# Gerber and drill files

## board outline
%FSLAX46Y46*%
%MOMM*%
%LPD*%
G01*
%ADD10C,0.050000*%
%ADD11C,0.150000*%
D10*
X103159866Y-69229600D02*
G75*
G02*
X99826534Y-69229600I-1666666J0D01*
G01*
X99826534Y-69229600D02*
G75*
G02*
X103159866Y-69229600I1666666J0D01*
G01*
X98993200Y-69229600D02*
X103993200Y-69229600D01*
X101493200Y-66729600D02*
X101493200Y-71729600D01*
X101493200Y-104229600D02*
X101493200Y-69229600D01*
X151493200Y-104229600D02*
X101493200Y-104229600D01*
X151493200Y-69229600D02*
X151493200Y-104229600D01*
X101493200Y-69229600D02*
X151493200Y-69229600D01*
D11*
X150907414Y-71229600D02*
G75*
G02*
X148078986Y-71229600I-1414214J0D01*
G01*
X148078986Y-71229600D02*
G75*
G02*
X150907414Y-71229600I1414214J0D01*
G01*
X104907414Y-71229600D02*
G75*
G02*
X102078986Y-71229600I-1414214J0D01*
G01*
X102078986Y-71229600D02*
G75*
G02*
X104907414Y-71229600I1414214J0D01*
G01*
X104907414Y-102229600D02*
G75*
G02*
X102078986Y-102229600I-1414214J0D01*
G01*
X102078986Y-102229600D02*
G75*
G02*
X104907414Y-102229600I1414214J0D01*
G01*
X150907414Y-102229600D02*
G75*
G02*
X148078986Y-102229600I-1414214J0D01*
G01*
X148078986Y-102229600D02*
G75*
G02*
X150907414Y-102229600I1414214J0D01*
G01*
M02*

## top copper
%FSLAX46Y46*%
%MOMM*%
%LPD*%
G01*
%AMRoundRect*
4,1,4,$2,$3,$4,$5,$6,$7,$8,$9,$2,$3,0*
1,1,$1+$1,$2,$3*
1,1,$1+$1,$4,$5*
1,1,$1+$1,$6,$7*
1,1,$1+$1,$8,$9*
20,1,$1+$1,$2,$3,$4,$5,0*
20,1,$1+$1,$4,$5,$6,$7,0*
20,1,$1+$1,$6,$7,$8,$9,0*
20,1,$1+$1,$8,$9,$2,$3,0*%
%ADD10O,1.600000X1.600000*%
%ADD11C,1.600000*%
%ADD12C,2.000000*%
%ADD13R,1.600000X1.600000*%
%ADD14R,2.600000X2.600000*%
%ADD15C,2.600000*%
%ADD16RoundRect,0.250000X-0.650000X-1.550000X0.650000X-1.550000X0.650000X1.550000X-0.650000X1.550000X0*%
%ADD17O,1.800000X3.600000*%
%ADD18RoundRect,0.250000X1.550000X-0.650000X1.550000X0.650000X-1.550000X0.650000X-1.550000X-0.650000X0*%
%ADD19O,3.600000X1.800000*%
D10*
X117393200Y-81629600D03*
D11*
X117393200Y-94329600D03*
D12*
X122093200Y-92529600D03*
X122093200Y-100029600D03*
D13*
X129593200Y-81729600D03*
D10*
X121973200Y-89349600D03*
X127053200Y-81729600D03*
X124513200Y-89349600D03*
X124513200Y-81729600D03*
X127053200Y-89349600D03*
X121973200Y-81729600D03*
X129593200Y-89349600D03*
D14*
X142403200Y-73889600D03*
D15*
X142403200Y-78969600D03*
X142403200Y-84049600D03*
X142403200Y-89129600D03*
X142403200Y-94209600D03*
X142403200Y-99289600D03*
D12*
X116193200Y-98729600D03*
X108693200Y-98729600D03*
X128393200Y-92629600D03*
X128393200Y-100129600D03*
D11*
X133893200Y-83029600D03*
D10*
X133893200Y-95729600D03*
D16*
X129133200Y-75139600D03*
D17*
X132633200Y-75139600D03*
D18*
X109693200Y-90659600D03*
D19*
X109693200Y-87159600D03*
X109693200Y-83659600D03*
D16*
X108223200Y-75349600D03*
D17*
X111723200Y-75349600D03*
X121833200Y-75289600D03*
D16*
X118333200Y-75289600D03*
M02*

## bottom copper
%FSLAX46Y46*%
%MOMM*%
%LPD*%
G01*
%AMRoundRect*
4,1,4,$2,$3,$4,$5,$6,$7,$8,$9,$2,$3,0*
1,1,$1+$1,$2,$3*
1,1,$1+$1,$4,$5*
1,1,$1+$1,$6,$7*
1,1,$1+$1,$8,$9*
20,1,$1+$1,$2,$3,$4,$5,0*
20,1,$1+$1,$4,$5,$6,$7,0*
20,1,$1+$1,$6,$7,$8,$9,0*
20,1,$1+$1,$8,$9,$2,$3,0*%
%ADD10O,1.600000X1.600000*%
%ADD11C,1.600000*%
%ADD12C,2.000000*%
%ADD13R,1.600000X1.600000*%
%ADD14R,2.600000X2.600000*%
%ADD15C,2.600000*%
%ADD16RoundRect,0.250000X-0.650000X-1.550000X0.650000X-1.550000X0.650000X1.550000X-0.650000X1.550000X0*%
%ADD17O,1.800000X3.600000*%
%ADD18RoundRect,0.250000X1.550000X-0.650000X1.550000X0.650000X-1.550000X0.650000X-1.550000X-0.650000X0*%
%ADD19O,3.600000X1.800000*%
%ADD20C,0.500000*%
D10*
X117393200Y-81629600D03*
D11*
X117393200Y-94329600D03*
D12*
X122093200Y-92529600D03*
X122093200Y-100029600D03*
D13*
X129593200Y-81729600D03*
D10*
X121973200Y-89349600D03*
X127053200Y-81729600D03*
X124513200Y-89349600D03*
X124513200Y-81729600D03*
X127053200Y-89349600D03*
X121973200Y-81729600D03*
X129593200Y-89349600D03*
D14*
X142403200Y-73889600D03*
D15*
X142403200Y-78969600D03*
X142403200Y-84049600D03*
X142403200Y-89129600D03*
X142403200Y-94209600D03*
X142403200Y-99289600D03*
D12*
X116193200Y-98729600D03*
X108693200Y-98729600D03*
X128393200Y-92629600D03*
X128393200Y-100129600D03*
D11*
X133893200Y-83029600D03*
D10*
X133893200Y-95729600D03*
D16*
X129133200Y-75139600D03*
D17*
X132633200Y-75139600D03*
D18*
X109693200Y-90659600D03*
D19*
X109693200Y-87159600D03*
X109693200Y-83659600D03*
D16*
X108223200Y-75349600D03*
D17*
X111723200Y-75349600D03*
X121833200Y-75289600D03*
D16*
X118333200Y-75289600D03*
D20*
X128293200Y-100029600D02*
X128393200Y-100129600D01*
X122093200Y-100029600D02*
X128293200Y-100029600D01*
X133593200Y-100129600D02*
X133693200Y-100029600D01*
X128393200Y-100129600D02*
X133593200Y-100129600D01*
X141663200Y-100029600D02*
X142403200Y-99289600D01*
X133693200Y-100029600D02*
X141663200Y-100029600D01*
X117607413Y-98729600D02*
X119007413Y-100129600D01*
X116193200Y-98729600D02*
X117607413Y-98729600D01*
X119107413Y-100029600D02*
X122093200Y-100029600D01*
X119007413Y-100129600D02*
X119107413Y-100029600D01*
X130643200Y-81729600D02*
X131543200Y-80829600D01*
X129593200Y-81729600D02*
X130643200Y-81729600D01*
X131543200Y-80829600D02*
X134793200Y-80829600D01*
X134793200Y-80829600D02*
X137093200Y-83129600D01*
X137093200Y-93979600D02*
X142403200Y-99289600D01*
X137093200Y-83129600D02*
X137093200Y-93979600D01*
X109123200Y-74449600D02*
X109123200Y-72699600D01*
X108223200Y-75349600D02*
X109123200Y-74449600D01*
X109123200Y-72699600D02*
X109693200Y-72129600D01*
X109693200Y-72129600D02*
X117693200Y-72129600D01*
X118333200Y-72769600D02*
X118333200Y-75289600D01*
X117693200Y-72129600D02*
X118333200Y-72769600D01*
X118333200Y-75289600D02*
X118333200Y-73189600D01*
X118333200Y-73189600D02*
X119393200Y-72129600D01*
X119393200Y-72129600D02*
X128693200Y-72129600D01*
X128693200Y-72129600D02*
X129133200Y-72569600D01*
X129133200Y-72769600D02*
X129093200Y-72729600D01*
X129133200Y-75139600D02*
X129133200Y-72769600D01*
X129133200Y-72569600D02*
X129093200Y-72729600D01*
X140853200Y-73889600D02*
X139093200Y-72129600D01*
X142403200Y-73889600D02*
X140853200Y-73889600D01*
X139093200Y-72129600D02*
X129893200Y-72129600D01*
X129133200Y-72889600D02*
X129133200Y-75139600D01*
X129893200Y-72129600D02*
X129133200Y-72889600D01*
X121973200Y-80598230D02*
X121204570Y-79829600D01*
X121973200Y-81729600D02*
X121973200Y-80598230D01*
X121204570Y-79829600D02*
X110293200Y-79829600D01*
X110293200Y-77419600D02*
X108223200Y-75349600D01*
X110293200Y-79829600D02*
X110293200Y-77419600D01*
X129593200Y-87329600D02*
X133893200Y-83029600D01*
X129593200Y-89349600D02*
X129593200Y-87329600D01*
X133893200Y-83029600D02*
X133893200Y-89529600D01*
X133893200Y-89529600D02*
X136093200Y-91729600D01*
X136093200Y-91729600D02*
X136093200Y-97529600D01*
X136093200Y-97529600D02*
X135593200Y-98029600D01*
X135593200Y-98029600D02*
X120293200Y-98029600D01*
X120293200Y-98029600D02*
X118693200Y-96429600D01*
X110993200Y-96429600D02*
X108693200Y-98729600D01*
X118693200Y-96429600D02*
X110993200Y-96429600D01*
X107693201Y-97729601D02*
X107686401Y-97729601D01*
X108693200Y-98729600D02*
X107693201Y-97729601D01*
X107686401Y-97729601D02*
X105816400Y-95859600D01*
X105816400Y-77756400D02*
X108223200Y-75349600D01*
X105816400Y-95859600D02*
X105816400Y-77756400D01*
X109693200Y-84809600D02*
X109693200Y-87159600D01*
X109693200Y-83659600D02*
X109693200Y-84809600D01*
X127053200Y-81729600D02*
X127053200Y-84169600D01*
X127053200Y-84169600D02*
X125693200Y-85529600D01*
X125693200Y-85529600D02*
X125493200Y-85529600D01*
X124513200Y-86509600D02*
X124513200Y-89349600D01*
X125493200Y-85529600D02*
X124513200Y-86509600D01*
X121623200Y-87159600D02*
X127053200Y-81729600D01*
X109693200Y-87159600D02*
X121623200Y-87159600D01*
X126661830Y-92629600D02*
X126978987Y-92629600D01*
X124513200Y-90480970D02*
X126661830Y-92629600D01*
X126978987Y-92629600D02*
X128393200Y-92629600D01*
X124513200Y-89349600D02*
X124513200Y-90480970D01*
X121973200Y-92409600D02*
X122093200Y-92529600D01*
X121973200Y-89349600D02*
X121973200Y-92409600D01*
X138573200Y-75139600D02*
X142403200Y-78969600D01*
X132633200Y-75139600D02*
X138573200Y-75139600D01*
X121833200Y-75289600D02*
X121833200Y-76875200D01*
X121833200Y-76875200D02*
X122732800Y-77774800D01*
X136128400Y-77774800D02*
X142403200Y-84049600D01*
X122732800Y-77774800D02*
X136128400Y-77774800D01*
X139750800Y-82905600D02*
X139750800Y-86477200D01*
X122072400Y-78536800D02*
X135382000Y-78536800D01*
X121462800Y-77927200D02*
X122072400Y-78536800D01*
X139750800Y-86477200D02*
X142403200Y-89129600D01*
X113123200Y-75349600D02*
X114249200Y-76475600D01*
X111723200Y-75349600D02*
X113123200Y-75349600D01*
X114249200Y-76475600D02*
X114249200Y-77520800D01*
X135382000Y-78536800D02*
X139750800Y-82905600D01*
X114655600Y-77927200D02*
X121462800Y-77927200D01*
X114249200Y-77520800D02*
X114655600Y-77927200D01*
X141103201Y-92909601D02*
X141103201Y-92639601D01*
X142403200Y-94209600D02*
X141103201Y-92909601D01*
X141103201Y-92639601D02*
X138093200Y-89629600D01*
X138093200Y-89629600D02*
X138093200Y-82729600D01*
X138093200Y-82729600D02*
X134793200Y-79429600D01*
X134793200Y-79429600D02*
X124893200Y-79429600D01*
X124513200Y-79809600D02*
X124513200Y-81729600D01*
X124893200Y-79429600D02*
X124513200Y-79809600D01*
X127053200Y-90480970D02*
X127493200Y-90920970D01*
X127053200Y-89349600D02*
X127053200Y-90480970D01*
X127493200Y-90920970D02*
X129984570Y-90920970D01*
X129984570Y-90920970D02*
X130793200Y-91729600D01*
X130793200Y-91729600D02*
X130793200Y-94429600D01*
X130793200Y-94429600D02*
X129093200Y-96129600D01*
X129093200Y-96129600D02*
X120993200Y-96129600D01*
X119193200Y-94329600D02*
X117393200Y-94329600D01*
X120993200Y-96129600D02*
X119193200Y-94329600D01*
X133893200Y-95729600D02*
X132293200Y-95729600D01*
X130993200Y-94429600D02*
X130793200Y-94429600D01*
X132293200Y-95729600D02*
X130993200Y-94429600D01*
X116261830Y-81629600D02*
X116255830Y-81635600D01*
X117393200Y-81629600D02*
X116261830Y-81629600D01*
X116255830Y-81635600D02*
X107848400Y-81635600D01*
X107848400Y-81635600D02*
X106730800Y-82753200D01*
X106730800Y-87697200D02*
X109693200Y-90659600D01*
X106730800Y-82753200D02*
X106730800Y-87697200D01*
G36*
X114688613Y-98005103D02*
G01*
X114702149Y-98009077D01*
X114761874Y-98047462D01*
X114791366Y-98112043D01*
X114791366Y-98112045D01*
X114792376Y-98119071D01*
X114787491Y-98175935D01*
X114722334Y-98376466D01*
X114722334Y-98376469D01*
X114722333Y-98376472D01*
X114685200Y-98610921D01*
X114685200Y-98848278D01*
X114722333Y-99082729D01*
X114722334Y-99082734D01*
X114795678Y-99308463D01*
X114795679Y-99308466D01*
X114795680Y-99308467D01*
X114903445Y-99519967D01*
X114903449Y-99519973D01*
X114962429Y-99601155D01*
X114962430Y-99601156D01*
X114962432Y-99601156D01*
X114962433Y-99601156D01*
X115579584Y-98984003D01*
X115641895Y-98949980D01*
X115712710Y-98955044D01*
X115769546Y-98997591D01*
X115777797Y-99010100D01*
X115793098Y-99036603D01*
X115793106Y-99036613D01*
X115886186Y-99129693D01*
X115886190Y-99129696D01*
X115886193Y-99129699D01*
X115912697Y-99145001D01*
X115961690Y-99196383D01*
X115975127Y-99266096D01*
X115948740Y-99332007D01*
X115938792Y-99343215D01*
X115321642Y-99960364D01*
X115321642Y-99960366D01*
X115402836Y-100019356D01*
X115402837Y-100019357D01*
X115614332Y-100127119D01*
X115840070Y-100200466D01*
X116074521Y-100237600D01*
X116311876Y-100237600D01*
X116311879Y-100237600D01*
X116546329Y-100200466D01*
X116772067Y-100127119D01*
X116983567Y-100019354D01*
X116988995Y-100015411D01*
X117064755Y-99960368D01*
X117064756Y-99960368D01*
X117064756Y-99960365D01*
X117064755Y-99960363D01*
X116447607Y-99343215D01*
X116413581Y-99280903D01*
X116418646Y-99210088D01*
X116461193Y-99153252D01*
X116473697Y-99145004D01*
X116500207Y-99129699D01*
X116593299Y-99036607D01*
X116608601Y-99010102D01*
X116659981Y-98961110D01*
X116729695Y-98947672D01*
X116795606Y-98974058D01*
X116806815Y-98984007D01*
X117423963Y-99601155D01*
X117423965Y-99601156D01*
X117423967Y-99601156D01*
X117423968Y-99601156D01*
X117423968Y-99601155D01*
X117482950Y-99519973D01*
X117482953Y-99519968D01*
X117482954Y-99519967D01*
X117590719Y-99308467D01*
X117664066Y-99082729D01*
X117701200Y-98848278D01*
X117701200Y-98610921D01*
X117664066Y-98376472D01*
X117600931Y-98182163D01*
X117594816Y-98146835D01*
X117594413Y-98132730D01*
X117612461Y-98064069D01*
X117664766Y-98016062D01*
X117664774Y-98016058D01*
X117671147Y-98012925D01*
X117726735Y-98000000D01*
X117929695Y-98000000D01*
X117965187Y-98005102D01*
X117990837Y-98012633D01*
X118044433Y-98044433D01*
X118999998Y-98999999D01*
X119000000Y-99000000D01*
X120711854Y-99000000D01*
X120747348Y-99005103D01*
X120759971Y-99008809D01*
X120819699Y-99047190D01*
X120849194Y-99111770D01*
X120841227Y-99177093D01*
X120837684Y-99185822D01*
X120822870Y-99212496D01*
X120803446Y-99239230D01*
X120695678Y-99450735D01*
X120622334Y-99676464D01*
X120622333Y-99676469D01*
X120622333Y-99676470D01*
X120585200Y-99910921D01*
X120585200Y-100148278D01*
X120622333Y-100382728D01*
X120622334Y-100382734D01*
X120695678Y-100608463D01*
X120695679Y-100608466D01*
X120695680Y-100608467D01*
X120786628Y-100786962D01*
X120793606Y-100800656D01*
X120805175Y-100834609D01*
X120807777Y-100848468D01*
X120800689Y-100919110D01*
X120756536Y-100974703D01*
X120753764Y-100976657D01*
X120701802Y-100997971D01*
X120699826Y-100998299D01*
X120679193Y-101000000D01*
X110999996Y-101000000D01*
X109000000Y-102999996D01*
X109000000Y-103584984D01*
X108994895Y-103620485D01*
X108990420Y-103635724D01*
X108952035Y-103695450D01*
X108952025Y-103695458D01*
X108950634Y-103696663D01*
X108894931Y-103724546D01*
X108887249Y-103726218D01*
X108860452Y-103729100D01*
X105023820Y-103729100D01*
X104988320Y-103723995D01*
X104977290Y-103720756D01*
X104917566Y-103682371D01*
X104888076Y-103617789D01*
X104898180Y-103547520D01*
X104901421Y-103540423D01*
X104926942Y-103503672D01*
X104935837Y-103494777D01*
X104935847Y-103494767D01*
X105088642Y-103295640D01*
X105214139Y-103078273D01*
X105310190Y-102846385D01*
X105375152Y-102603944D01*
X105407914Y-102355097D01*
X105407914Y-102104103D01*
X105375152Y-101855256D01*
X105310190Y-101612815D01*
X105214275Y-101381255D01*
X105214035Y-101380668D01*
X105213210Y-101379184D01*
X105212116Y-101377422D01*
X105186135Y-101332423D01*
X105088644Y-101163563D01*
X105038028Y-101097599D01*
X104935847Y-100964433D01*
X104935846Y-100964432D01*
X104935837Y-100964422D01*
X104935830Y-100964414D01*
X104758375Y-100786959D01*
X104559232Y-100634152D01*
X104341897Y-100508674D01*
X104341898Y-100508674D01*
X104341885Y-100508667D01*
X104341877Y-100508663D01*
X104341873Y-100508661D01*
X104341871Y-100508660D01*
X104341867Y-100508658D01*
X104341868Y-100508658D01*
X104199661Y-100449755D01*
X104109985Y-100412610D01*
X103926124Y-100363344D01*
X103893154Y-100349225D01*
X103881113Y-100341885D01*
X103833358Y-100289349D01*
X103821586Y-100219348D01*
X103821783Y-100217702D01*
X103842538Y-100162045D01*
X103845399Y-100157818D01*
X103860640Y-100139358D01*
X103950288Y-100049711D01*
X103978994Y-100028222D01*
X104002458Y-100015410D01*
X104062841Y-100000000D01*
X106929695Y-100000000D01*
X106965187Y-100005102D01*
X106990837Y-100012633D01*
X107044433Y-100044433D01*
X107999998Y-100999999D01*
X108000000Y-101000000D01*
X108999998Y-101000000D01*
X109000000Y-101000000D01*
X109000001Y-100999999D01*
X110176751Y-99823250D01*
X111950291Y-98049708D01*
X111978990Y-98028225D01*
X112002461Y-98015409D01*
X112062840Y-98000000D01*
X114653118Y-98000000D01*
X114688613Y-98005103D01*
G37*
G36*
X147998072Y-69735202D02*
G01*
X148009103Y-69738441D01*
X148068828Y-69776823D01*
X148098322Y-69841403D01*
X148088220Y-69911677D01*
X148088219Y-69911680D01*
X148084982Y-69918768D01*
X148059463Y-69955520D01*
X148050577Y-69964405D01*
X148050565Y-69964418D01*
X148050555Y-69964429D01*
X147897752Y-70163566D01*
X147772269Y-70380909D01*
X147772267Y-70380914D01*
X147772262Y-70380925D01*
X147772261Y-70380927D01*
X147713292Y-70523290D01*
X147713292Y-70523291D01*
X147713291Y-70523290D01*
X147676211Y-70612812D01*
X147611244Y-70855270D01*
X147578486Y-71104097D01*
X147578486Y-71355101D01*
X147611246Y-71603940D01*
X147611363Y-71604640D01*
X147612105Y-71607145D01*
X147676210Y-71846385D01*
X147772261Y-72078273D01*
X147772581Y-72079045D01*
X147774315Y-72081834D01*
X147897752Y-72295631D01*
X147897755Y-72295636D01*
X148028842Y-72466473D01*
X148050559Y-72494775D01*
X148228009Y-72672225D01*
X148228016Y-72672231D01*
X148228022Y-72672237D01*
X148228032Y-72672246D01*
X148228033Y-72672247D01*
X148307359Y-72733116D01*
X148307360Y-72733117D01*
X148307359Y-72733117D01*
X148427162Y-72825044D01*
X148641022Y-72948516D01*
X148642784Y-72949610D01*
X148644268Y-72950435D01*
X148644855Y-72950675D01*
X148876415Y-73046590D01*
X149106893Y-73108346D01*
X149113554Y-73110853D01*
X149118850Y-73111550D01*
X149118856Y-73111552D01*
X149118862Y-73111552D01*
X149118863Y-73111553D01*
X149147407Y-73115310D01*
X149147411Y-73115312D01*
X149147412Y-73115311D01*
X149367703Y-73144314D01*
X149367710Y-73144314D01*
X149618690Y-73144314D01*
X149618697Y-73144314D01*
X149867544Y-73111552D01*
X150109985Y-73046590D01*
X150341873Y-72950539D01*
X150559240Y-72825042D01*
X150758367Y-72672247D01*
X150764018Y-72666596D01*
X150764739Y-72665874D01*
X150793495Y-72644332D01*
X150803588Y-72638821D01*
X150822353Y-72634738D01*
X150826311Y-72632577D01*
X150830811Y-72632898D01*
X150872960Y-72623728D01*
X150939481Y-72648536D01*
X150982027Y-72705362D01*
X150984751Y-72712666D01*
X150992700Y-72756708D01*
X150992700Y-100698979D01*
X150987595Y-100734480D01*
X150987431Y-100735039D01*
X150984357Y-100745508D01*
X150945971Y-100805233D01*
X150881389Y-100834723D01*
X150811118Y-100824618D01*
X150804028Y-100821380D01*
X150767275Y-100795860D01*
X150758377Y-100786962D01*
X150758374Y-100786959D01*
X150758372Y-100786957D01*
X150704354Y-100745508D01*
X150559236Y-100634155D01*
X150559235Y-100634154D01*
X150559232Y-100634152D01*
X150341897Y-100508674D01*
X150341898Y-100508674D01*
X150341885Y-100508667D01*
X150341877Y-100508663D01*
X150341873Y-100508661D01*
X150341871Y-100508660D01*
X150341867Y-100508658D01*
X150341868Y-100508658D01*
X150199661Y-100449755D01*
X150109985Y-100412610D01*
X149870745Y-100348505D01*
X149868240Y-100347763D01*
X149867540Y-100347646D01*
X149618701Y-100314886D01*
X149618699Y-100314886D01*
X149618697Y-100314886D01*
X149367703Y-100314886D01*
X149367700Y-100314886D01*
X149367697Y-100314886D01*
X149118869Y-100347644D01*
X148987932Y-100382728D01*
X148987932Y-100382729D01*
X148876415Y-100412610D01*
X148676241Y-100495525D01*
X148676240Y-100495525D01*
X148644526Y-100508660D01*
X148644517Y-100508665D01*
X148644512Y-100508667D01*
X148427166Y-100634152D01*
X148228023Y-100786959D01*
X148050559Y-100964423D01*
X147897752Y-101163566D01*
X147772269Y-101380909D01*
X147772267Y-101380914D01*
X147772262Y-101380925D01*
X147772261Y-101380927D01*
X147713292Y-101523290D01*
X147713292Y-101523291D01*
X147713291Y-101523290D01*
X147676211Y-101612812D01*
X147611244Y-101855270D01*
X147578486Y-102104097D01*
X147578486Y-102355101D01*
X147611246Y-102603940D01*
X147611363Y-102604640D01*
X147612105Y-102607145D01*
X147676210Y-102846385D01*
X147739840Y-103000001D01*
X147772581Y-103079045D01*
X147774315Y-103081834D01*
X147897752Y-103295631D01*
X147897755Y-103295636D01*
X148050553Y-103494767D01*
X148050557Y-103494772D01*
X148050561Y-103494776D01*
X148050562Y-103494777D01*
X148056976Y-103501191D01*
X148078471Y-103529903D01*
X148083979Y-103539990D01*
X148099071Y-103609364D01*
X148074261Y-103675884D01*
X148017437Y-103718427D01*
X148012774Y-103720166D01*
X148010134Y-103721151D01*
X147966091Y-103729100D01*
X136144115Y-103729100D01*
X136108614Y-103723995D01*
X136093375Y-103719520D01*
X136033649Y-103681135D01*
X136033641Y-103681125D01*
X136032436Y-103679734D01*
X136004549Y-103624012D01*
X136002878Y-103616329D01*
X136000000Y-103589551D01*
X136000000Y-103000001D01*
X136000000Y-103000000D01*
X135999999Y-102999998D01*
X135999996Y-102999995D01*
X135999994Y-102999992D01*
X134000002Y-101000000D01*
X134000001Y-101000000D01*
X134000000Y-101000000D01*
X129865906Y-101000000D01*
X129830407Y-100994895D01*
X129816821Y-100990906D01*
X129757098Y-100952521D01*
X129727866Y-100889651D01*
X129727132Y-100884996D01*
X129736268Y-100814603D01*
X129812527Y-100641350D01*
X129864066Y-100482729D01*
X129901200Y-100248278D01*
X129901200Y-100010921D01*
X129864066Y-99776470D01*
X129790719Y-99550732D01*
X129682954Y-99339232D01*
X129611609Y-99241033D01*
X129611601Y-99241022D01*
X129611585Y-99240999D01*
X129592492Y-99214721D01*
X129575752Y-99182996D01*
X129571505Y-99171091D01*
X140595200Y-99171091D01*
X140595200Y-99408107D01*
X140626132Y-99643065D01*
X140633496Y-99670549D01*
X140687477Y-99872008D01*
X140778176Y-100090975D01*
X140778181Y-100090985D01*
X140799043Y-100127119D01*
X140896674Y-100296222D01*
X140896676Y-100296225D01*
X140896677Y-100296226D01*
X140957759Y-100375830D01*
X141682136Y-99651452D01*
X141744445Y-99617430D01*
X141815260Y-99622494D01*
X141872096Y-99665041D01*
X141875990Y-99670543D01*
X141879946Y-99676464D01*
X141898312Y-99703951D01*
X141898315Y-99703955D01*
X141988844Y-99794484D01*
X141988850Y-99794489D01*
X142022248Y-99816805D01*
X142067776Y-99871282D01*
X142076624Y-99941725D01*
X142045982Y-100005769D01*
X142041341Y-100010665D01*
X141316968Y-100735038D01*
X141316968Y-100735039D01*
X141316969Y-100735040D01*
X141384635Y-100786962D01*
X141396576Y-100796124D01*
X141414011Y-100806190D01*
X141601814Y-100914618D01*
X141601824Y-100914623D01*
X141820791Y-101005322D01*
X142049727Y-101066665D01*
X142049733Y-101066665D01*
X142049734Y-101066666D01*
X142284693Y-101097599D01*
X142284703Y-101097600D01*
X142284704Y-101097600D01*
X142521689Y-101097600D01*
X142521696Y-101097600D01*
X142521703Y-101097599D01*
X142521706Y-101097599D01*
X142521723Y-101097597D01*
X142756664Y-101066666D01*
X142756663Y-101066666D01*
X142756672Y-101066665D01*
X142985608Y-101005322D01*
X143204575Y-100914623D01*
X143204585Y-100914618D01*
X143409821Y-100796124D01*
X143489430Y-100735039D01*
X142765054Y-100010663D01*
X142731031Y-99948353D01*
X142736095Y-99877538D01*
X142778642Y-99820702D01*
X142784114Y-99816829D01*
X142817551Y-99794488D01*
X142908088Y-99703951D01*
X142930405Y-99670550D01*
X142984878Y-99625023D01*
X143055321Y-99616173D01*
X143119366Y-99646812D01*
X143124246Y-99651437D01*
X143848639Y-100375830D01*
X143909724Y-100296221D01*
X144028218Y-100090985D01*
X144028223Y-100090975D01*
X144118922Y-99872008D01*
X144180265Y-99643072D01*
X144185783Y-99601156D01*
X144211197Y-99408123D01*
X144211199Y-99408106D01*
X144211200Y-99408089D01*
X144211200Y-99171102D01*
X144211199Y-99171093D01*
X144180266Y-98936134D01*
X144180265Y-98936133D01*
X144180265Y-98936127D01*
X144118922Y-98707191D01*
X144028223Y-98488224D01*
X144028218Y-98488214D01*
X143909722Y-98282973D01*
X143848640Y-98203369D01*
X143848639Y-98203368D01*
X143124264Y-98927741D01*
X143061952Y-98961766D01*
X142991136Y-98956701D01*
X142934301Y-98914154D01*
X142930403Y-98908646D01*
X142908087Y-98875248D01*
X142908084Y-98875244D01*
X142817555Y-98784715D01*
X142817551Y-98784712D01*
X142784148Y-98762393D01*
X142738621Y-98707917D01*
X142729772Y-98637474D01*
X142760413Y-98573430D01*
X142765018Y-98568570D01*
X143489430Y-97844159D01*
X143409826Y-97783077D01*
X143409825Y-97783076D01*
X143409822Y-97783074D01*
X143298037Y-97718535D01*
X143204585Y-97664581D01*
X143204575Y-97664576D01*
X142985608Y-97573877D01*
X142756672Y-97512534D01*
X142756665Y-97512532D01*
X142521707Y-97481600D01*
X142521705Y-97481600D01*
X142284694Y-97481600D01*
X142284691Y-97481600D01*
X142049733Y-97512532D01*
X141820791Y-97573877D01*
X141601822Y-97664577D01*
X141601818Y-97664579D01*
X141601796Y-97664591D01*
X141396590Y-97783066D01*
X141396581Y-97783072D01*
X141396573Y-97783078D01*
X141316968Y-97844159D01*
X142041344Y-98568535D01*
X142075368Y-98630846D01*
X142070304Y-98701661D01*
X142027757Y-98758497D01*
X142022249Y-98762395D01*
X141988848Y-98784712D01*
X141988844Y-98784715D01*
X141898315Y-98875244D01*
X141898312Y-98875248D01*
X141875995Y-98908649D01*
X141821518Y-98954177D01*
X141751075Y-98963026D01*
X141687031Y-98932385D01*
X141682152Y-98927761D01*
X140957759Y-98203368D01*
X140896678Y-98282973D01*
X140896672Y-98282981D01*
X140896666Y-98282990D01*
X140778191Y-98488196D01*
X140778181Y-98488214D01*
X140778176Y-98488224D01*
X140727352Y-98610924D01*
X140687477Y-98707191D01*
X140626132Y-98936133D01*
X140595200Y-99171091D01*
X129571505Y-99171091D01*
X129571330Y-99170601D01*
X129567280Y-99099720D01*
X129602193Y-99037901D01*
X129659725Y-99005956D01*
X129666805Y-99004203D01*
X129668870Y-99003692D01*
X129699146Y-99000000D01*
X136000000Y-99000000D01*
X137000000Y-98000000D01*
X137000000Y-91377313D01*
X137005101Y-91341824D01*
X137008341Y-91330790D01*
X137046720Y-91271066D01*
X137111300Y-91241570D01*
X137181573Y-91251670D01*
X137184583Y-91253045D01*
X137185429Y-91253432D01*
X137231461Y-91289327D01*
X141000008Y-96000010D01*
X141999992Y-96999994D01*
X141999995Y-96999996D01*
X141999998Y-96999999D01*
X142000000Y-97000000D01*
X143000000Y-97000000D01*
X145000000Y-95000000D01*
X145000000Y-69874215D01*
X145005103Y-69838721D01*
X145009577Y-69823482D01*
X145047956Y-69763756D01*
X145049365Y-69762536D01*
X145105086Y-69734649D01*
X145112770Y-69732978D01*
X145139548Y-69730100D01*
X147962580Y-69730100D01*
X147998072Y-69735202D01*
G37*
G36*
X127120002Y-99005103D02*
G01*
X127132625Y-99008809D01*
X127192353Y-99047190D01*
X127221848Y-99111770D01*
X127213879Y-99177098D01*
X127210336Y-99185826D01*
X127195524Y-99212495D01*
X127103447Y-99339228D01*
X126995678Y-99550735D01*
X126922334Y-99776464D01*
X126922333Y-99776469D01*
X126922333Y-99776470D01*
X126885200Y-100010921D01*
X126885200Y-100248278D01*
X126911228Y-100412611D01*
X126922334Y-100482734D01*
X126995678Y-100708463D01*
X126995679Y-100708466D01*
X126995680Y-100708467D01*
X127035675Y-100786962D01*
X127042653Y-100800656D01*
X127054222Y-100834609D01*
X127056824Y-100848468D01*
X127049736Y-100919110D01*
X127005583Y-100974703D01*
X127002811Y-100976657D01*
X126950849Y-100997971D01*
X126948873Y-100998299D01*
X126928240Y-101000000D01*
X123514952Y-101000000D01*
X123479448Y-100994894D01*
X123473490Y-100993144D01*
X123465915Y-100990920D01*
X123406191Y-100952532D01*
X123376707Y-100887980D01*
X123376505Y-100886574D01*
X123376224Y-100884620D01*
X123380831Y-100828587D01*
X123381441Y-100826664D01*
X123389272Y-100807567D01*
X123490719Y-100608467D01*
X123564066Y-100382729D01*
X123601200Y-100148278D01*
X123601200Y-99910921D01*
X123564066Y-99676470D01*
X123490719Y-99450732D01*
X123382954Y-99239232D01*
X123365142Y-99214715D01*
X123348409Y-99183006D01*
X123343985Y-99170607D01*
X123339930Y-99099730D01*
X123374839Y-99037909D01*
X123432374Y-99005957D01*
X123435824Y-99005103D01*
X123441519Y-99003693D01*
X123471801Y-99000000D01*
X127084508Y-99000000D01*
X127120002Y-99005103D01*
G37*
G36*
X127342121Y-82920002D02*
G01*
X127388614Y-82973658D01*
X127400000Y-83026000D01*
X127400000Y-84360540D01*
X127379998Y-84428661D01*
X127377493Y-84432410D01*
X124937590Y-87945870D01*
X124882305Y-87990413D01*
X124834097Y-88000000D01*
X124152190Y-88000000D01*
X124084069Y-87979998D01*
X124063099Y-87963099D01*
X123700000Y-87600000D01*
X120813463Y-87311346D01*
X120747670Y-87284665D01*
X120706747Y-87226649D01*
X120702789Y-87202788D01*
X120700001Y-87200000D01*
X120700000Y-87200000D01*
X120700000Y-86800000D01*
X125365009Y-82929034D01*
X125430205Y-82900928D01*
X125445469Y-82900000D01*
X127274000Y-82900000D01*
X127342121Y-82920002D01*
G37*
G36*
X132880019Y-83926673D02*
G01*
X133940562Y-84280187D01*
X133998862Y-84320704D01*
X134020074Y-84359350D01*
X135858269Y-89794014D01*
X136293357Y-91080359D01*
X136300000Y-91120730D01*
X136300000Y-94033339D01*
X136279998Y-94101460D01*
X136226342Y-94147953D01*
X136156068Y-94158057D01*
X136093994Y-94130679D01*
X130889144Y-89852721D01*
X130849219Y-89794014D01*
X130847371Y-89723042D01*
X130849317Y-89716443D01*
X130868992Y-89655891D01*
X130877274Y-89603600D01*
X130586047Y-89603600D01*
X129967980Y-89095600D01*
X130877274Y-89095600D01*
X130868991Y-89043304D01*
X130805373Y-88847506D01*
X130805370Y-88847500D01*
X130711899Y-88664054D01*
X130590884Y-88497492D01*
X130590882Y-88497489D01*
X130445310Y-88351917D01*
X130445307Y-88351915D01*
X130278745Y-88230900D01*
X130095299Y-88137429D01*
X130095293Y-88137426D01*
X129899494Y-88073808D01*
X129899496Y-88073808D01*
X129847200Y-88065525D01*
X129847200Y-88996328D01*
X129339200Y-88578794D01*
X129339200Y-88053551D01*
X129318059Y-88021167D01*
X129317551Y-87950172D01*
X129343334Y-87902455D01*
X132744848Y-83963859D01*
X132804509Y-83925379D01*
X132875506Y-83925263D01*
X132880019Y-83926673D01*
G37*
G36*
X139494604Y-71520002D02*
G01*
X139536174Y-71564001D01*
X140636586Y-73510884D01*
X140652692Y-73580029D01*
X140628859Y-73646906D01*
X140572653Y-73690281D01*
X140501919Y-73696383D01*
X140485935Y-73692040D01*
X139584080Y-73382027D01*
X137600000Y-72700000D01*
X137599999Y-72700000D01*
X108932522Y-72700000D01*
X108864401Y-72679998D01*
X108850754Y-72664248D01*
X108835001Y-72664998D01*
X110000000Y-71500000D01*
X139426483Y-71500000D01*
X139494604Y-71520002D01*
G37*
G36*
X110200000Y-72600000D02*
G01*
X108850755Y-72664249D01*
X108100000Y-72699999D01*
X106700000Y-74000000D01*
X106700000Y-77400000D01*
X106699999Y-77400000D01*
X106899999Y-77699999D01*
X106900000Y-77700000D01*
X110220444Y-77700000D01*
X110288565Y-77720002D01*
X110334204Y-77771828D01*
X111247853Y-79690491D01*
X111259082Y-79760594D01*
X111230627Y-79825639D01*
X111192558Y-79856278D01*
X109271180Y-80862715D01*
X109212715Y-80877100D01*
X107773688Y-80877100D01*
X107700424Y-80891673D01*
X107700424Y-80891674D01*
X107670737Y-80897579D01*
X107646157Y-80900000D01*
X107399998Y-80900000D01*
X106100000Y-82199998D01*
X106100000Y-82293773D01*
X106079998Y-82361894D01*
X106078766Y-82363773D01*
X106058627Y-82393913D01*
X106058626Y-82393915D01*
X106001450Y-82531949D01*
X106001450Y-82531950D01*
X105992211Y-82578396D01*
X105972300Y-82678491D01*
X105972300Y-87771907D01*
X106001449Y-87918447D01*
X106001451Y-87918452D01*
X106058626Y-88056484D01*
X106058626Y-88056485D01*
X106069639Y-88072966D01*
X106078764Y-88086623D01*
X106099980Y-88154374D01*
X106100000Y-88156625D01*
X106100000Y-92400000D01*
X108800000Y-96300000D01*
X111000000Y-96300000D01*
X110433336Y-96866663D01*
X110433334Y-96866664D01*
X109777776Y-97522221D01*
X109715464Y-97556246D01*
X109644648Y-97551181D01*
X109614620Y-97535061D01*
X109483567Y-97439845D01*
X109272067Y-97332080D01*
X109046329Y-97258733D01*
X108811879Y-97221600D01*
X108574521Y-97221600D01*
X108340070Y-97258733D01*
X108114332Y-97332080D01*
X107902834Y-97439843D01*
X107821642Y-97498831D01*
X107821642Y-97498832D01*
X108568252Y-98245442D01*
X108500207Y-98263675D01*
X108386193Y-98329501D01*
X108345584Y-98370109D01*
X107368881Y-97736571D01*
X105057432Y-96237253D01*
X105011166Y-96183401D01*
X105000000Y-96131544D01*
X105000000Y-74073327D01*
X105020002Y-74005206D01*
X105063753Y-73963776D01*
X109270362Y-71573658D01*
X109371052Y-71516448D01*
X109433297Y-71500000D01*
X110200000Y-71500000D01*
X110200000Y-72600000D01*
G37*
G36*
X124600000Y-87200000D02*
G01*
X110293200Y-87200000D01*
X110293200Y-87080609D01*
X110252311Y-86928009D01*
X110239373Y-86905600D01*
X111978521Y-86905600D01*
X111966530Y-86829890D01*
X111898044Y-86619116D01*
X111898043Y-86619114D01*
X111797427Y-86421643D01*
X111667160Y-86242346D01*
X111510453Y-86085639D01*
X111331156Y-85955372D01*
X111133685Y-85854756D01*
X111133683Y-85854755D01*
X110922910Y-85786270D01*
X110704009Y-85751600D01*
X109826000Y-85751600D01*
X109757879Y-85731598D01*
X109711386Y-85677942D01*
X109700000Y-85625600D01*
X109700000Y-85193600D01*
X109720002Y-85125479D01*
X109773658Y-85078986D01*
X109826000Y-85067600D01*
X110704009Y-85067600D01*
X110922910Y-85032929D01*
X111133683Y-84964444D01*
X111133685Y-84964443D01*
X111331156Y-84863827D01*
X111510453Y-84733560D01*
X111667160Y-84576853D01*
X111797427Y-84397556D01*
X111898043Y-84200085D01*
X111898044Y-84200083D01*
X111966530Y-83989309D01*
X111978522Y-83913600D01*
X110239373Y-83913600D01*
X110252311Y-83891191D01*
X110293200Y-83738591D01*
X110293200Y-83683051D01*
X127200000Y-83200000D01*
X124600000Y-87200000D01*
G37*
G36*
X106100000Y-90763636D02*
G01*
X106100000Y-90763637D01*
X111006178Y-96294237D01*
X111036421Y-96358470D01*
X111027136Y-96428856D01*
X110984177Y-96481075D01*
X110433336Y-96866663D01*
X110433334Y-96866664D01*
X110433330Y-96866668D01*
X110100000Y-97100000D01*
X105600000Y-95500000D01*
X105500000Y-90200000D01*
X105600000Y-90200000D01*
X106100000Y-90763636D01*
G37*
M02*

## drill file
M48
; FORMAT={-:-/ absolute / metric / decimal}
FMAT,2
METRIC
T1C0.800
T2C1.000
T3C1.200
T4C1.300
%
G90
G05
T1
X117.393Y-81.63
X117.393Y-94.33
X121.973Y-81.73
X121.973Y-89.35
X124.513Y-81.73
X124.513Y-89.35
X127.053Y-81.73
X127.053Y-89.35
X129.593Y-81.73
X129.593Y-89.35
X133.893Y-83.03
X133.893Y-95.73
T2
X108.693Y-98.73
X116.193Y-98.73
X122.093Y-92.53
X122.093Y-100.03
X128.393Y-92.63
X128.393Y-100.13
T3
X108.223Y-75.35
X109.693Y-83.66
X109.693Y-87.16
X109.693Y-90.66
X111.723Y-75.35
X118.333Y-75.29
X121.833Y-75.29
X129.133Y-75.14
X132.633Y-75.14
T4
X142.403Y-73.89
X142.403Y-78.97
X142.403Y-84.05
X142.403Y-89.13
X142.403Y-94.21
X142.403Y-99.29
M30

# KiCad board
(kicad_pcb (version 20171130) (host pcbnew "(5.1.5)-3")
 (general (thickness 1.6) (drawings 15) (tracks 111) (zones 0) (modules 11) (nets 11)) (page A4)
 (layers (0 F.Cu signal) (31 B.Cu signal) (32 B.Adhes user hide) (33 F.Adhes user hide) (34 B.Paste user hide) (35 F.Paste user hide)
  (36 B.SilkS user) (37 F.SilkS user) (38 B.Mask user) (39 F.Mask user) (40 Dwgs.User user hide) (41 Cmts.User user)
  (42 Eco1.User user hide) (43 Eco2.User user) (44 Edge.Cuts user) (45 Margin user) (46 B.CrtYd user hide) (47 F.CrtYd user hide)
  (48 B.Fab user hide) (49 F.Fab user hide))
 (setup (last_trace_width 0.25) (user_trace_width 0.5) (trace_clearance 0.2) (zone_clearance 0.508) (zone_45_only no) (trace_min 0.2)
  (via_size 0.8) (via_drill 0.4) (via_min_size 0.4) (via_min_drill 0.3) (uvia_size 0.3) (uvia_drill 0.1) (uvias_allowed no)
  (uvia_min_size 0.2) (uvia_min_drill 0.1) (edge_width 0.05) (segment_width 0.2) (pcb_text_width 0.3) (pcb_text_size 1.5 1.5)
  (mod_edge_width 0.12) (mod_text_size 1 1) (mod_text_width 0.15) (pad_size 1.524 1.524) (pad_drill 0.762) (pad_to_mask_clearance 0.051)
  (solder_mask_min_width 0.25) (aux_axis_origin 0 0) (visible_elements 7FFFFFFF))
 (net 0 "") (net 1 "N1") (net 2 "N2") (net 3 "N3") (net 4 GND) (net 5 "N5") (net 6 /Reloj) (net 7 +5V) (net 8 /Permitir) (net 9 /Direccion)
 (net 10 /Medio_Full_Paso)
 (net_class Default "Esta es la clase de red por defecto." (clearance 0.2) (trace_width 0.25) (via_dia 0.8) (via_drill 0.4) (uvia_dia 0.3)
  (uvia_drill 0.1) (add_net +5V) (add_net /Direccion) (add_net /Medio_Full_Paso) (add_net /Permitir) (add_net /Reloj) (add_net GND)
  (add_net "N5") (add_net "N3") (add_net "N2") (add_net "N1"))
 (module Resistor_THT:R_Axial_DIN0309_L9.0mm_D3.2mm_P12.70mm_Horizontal (layer F.Cu) (at 117.3932 94.3296 90)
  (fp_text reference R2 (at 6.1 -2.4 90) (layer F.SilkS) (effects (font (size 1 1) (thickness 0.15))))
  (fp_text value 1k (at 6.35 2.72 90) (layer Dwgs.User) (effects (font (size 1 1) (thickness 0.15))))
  (pad 2 thru_hole oval (at 12.7 0 90) (size 1.6 1.6) (drill 0.8) (layers *.Cu *.Mask) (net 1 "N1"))
  (pad 1 thru_hole circle (at 0 0 90) (size 1.6 1.6) (drill 0.8) (layers *.Cu *.Mask) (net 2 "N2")))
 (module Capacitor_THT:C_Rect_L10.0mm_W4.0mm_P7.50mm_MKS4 (layer F.Cu) (at 122.0932 92.5296 270)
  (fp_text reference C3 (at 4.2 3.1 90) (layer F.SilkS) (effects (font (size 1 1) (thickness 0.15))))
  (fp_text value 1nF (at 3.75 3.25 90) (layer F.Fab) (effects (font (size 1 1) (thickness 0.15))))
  (pad 1 thru_hole circle (at 0 0 270) (size 2 2) (drill 1) (layers *.Cu *.Mask) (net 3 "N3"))
  (pad 2 thru_hole circle (at 7.5 0 270) (size 2 2) (drill 1) (layers *.Cu *.Mask) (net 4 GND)))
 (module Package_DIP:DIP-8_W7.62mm (layer F.Cu) (at 129.5932 81.7296 270)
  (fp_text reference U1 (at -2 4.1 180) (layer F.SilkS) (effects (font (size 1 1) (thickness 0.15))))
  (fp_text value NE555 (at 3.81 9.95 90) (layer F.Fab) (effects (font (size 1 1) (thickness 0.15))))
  (pad 1 thru_hole rect (at 0 0 270) (size 1.6 1.6) (drill 0.8) (layers *.Cu *.Mask) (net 4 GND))
  (pad 5 thru_hole oval (at 7.62 7.62 270) (size 1.6 1.6) (drill 0.8) (layers *.Cu *.Mask) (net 3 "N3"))
  (pad 2 thru_hole oval (at 0 2.54 270) (size 1.6 1.6) (drill 0.8) (layers *.Cu *.Mask) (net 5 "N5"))
  (pad 6 thru_hole oval (at 7.62 5.08 270) (size 1.6 1.6) (drill 0.8) (layers *.Cu *.Mask) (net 5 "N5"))
  (pad 3 thru_hole oval (at 0 5.08 270) (size 1.6 1.6) (drill 0.8) (layers *.Cu *.Mask) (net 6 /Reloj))
  (pad 7 thru_hole oval (at 7.62 2.54 270) (size 1.6 1.6) (drill 0.8) (layers *.Cu *.Mask) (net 2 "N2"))
  (pad 4 thru_hole oval (at 0 7.62 270) (size 1.6 1.6) (drill 0.8) (layers *.Cu *.Mask) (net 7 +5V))
  (pad 8 thru_hole oval (at 7.62 0 270) (size 1.6 1.6) (drill 0.8) (layers *.Cu *.Mask) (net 7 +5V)))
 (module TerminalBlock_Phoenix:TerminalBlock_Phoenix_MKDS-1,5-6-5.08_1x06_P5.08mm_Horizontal (layer F.Cu) (at 142.4032 73.8896 270)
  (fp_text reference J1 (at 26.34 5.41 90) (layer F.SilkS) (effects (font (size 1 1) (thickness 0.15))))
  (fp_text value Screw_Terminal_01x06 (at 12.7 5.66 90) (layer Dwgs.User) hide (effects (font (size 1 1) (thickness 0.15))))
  (pad 1 thru_hole rect (at 0 0 270) (size 2.6 2.6) (drill 1.3) (layers *.Cu *.Mask) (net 7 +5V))
  (pad 2 thru_hole circle (at 5.08 0 270) (size 2.6 2.6) (drill 1.3) (layers *.Cu *.Mask) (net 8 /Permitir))
  (pad 3 thru_hole circle (at 10.16 0 270) (size 2.6 2.6) (drill 1.3) (layers *.Cu *.Mask) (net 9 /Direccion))
  (pad 4 thru_hole circle (at 15.24 0 270) (size 2.6 2.6) (drill 1.3) (layers *.Cu *.Mask) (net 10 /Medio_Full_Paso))
  (pad 5 thru_hole circle (at 20.32 0 270) (size 2.6 2.6) (drill 1.3) (layers *.Cu *.Mask) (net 6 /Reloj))
  (pad 6 thru_hole circle (at 25.4 0 270) (size 2.6 2.6) (drill 1.3) (layers *.Cu *.Mask) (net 4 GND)))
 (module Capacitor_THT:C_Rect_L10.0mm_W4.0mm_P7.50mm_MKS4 (layer F.Cu) (at 108.6932 98.7296)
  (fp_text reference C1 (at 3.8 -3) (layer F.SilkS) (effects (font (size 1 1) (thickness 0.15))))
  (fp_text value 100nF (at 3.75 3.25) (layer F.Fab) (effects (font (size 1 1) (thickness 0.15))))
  (pad 2 thru_hole circle (at 7.5 0) (size 2 2) (drill 1) (layers *.Cu *.Mask) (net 4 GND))
  (pad 1 thru_hole circle (at 0 0) (size 2 2) (drill 1) (layers *.Cu *.Mask) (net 7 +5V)))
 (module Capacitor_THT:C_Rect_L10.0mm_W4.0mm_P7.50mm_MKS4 (layer F.Cu) (at 128.3932 92.6296 270)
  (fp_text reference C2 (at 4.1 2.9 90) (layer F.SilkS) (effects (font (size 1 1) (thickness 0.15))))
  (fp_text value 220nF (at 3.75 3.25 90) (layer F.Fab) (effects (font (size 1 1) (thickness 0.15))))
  (pad 1 thru_hole circle (at 0 0 270) (size 2 2) (drill 1) (layers *.Cu *.Mask) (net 5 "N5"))
  (pad 2 thru_hole circle (at 7.5 0 270) (size 2 2) (drill 1) (layers *.Cu *.Mask) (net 4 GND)))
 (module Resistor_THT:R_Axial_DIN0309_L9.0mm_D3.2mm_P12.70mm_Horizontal (layer F.Cu) (at 133.8932 83.0296 270)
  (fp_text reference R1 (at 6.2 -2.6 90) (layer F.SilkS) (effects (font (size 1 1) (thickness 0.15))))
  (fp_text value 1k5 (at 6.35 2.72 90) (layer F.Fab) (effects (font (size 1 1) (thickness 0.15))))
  (pad 1 thru_hole circle (at 0 0 270) (size 1.6 1.6) (drill 0.8) (layers *.Cu *.Mask) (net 7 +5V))
  (pad 2 thru_hole oval (at 12.7 0 270) (size 1.6 1.6) (drill 0.8) (layers *.Cu *.Mask) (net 2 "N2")))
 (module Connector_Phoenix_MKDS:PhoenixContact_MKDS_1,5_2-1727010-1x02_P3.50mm (layer F.Cu) (at 129.1332 72.5996)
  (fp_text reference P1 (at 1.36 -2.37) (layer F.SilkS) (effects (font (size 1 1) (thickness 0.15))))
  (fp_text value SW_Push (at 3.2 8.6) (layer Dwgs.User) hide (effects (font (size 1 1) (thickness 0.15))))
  (pad 1 thru_hole roundrect (at 0 2.54) (size 1.8 3.6) (drill 1.2) (layers *.Cu *.Mask) (roundrect_rratio 0.138889) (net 7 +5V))
  (pad 2 thru_hole oval (at 3.5 2.54) (size 1.8 3.6) (drill 1.2) (layers *.Cu *.Mask) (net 8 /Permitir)))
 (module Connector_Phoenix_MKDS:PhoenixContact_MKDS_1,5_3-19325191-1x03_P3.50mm (layer F.Cu) (at 107.1532 90.6596 90)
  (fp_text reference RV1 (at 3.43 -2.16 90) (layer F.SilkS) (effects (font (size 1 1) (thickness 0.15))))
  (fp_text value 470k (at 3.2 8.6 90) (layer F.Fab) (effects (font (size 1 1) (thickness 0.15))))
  (pad 1 thru_hole roundrect (at 0 2.54 90) (size 1.8 3.6) (drill 1.2) (layers *.Cu *.Mask) (roundrect_rratio 0.138889) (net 1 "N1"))
  (pad 2 thru_hole oval (at 3.5 2.54 90) (size 1.8 3.6) (drill 1.2) (layers *.Cu *.Mask) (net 5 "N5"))
  (pad 3 thru_hole oval (at 7 2.54 90) (size 1.8 3.6) (drill 1.2) (layers *.Cu *.Mask) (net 5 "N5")))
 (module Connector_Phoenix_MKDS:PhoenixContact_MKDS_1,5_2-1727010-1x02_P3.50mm (layer F.Cu) (at 108.2232 72.8096)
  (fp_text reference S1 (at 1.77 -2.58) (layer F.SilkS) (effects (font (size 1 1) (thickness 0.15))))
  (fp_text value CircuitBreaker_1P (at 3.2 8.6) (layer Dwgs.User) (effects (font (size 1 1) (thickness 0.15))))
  (pad 1 thru_hole roundrect (at 0 2.54) (size 1.8 3.6) (drill 1.2) (layers *.Cu *.Mask) (roundrect_rratio 0.138889) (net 7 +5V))
  (pad 2 thru_hole oval (at 3.5 2.54) (size 1.8 3.6) (drill 1.2) (layers *.Cu *.Mask) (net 10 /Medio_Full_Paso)))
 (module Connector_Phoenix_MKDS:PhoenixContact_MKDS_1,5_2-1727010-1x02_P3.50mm (layer F.Cu) (at 118.3332 72.7496)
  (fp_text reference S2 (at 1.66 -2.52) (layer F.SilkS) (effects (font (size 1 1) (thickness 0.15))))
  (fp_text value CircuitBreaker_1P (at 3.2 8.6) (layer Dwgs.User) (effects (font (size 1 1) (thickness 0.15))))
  (pad 2 thru_hole oval (at 3.5 2.54) (size 1.8 3.6) (drill 1.2) (layers *.Cu *.Mask) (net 9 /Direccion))
  (pad 1 thru_hole roundrect (at 0 2.54) (size 1.8 3.6) (drill 1.2) (layers *.Cu *.Mask) (roundrect_rratio 0.138889) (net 7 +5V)))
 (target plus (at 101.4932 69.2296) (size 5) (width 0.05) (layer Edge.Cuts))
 (gr_line (start 101.4932 104.2296) (end 101.4932 69.2296) (layer Edge.Cuts) (width 0.05))
 (gr_line (start 151.4932 104.2296) (end 101.4932 104.2296) (layer Edge.Cuts) (width 0.05))
 (gr_line (start 151.4932 69.2296) (end 151.4932 104.2296) (layer Edge.Cuts) (width 0.05))
 (gr_line (start 101.4932 69.2296) (end 151.4932 69.2296) (layer Edge.Cuts) (width 0.05))
 (gr_circle (center 149.4932 71.2296) (end 150.907414 71.2296) (layer Edge.Cuts) (width 0.15))
 (gr_circle (center 103.4932 71.2296) (end 104.907414 71.2296) (layer Edge.Cuts) (width 0.15))
 (gr_circle (center 103.4932 102.2296) (end 104.907414 102.2296) (layer Edge.Cuts) (width 0.15))
 (gr_circle (center 149.4932 102.2296) (end 150.907414 102.2296) (layer Edge.Cuts) (width 0.15))
 (segment (start 128.2932 100.0296) (end 128.3932 100.1296) (width 0.5) (layer B.Cu) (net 4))
 (segment (start 122.0932 100.0296) (end 128.2932 100.0296) (width 0.5) (layer B.Cu) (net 4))
 (segment (start 133.5932 100.1296) (end 133.6932 100.0296) (width 0.5) (layer B.Cu) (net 4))
 (segment (start 128.3932 100.1296) (end 133.5932 100.1296) (width 0.5) (layer B.Cu) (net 4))
 (segment (start 141.6632 100.0296) (end 142.4032 99.2896) (width 0.5) (layer B.Cu) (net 4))
 (segment (start 133.6932 100.0296) (end 141.6632 100.0296) (width 0.5) (layer B.Cu) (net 4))
 (segment (start 117.607413 98.7296) (end 119.007413 100.1296) (width 0.5) (layer B.Cu) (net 4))
 (segment (start 116.1932 98.7296) (end 117.607413 98.7296) (width 0.5) (layer B.Cu) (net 4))
 (segment (start 119.107413 100.0296) (end 122.0932 100.0296) (width 0.5) (layer B.Cu) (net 4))
 (segment (start 119.007413 100.1296) (end 119.107413 100.0296) (width 0.5) (layer B.Cu) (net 4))
 (segment (start 130.6432 81.7296) (end 131.5432 80.8296) (width 0.5) (layer B.Cu) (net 4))
 (segment (start 129.5932 81.7296) (end 130.6432 81.7296) (width 0.5) (layer B.Cu) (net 4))
 (segment (start 131.5432 80.8296) (end 134.7932 80.8296) (width 0.5) (layer B.Cu) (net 4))
 (segment (start 134.7932 80.8296) (end 137.0932 83.1296) (width 0.5) (layer B.Cu) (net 4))
 (segment (start 137.0932 93.9796) (end 142.4032 99.2896) (width 0.5) (layer B.Cu) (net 4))
 (segment (start 137.0932 83.1296) (end 137.0932 93.9796) (width 0.5) (layer B.Cu) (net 4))
 (segment (start 109.1232 74.4496) (end 109.1232 72.6996) (width 0.5) (layer B.Cu) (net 7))
 (segment (start 108.2232 75.3496) (end 109.1232 74.4496) (width 0.5) (layer B.Cu) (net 7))
 (segment (start 109.1232 72.6996) (end 109.6932 72.1296) (width 0.5) (layer B.Cu) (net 7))
 (segment (start 109.6932 72.1296) (end 117.6932 72.1296) (width 0.5) (layer B.Cu) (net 7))
 (segment (start 118.3332 72.7696) (end 118.3332 75.2896) (width 0.5) (layer B.Cu) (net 7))
 (segment (start 117.6932 72.1296) (end 118.3332 72.7696) (width 0.5) (layer B.Cu) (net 7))
 (segment (start 118.3332 75.2896) (end 118.3332 73.1896) (width 0.5) (layer B.Cu) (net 7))
 (segment (start 118.3332 73.1896) (end 119.3932 72.1296) (width 0.5) (layer B.Cu) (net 7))
 (segment (start 119.3932 72.1296) (end 128.6932 72.1296) (width 0.5) (layer B.Cu) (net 7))
 (segment (start 128.6932 72.1296) (end 129.1332 72.5696) (width 0.5) (layer B.Cu) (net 7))
 (segment (start 129.1332 72.7696) (end 129.0932 72.7296) (width 0.5) (layer B.Cu) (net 7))
 (segment (start 129.1332 75.1396) (end 129.1332 72.7696) (width 0.5) (layer B.Cu) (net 7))
 (segment (start 129.1332 72.5696) (end 129.0932 72.7296) (width 0.5) (layer B.Cu) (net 7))
 (segment (start 140.8532 73.8896) (end 139.0932 72.1296) (width 0.5) (layer B.Cu) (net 7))
 (segment (start 142.4032 73.8896) (end 140.8532 73.8896) (width 0.5) (layer B.Cu) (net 7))
 (segment (start 139.0932 72.1296) (end 129.8932 72.1296) (width 0.5) (layer B.Cu) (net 7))
 (segment (start 129.1332 72.8896) (end 129.1332 75.1396) (width 0.5) (layer B.Cu) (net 7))
 (segment (start 129.8932 72.1296) (end 129.1332 72.8896) (width 0.5) (layer B.Cu) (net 7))
 (segment (start 121.9732 80.59823) (end 121.20457 79.8296) (width 0.5) (layer B.Cu) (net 7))
 (segment (start 121.9732 81.7296) (end 121.9732 80.59823) (width 0.5) (layer B.Cu) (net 7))
 (segment (start 121.20457 79.8296) (end 110.2932 79.8296) (width 0.5) (layer B.Cu) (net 7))
 (segment (start 110.2932 77.4196) (end 108.2232 75.3496) (width 0.5) (layer B.Cu) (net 7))
 (segment (start 110.2932 79.8296) (end 110.2932 77.4196) (width 0.5) (layer B.Cu) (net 7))
 (segment (start 129.5932 87.3296) (end 133.8932 83.0296) (width 0.5) (layer B.Cu) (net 7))
 (segment (start 129.5932 89.3496) (end 129.5932 87.3296) (width 0.5) (layer B.Cu) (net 7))
 (segment (start 133.8932 83.0296) (end 133.8932 89.5296) (width 0.5) (layer B.Cu) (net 7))
 (segment (start 133.8932 89.5296) (end 136.0932 91.7296) (width 0.5) (layer B.Cu) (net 7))
 (segment (start 136.0932 91.7296) (end 136.0932 97.5296) (width 0.5) (layer B.Cu) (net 7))
 (segment (start 136.0932 97.5296) (end 135.5932 98.0296) (width 0.5) (layer B.Cu) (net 7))
 (segment (start 135.5932 98.0296) (end 120.2932 98.0296) (width 0.5) (layer B.Cu) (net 7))
 (segment (start 120.2932 98.0296) (end 118.6932 96.4296) (width 0.5) (layer B.Cu) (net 7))
 (segment (start 110.9932 96.4296) (end 108.6932 98.7296) (width 0.5) (layer B.Cu) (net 7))
 (segment (start 118.6932 96.4296) (end 110.9932 96.4296) (width 0.5) (layer B.Cu) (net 7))
 (segment (start 107.693201 97.729601) (end 107.686401 97.729601) (width 0.5) (layer B.Cu) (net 7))
 (segment (start 108.6932 98.7296) (end 107.693201 97.729601) (width 0.5) (layer B.Cu) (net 7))
 (segment (start 107.686401 97.729601) (end 105.8164 95.8596) (width 0.5) (layer B.Cu) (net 7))
 (segment (start 105.8164 77.7564) (end 108.2232 75.3496) (width 0.5) (layer B.Cu) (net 7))
 (segment (start 105.8164 95.8596) (end 105.8164 77.7564) (width 0.5) (layer B.Cu) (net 7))
 (segment (start 109.6932 84.8096) (end 109.6932 87.1596) (width 0.5) (layer B.Cu) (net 5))
 (segment (start 109.6932 83.6596) (end 109.6932 84.8096) (width 0.5) (layer B.Cu) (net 5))
 (segment (start 127.0532 81.7296) (end 127.0532 84.1696) (width 0.5) (layer B.Cu) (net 5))
 (segment (start 127.0532 84.1696) (end 125.6932 85.5296) (width 0.5) (layer B.Cu) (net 5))
 (segment (start 125.6932 85.5296) (end 125.4932 85.5296) (width 0.5) (layer B.Cu) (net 5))
 (segment (start 124.5132 86.5096) (end 124.5132 89.3496) (width 0.5) (layer B.Cu) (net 5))
 (segment (start 125.4932 85.5296) (end 124.5132 86.5096) (width 0.5) (layer B.Cu) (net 5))
 (segment (start 121.6232 87.1596) (end 127.0532 81.7296) (width 0.5) (layer B.Cu) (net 5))
 (segment (start 109.6932 87.1596) (end 121.6232 87.1596) (width 0.5) (layer B.Cu) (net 5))
 (segment (start 126.66183 92.6296) (end 126.978987 92.6296) (width 0.5) (layer B.Cu) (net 5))
 (segment (start 124.5132 90.48097) (end 126.66183 92.6296) (width 0.5) (layer B.Cu) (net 5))
 (segment (start 126.978987 92.6296) (end 128.3932 92.6296) (width 0.5) (layer B.Cu) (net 5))
 (segment (start 124.5132 89.3496) (end 124.5132 90.48097) (width 0.5) (layer B.Cu) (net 5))
 (segment (start 121.9732 92.4096) (end 122.0932 92.5296) (width 0.5) (layer B.Cu) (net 3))
 (segment (start 121.9732 89.3496) (end 121.9732 92.4096) (width 0.5) (layer B.Cu) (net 3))
 (segment (start 138.5732 75.1396) (end 142.4032 78.9696) (width 0.5) (layer B.Cu) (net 8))
 (segment (start 132.6332 75.1396) (end 138.5732 75.1396) (width 0.5) (layer B.Cu) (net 8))
 (segment (start 121.8332 75.2896) (end 121.8332 76.8752) (width 0.5) (layer B.Cu) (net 9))
 (segment (start 121.8332 76.8752) (end 122.7328 77.7748) (width 0.5) (layer B.Cu) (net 9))
 (segment (start 136.1284 77.7748) (end 142.4032 84.0496) (width 0.5) (layer B.Cu) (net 9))
 (segment (start 122.7328 77.7748) (end 136.1284 77.7748) (width 0.5) (layer B.Cu) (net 9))
 (segment (start 139.7508 82.9056) (end 139.7508 86.4772) (width 0.5) (layer B.Cu) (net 10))
 (segment (start 122.0724 78.5368) (end 135.382 78.5368) (width 0.5) (layer B.Cu) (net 10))
 (segment (start 121.4628 77.9272) (end 122.0724 78.5368) (width 0.5) (layer B.Cu) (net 10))
 (segment (start 139.7508 86.4772) (end 142.4032 89.1296) (width 0.5) (layer B.Cu) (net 10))
 (segment (start 113.1232 75.3496) (end 114.2492 76.4756) (width 0.5) (layer B.Cu) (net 10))
 (segment (start 111.7232 75.3496) (end 113.1232 75.3496) (width 0.5) (layer B.Cu) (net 10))
 (segment (start 114.2492 76.4756) (end 114.2492 77.5208) (width 0.5) (layer B.Cu) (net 10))
 (segment (start 135.382 78.5368) (end 139.7508 82.9056) (width 0.5) (layer B.Cu) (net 10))
 (segment (start 114.6556 77.9272) (end 121.4628 77.9272) (width 0.5) (layer B.Cu) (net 10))
 (segment (start 114.2492 77.5208) (end 114.6556 77.9272) (width 0.5) (layer B.Cu) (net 10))
 (segment (start 141.103201 92.909601) (end 141.103201 92.639601) (width 0.5) (layer B.Cu) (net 6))
 (segment (start 142.4032 94.2096) (end 141.103201 92.909601) (width 0.5) (layer B.Cu) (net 6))
 (segment (start 141.103201 92.639601) (end 138.0932 89.6296) (width 0.5) (layer B.Cu) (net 6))
 (segment (start 138.0932 89.6296) (end 138.0932 82.7296) (width 0.5) (layer B.Cu) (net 6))
 (segment (start 138.0932 82.7296) (end 134.7932 79.4296) (width 0.5) (layer B.Cu) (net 6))
 (segment (start 134.7932 79.4296) (end 124.8932 79.4296) (width 0.5) (layer B.Cu) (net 6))
 (segment (start 124.5132 79.8096) (end 124.5132 81.7296) (width 0.5) (layer B.Cu) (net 6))
 (segment (start 124.8932 79.4296) (end 124.5132 79.8096) (width 0.5) (layer B.Cu) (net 6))
 (segment (start 127.0532 90.48097) (end 127.4932 90.92097) (width 0.5) (layer B.Cu) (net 2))
 (segment (start 127.0532 89.3496) (end 127.0532 90.48097) (width 0.5) (layer B.Cu) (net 2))
 (segment (start 127.4932 90.92097) (end 129.98457 90.92097) (width 0.5) (layer B.Cu) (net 2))
 (segment (start 129.98457 90.92097) (end 130.7932 91.7296) (width 0.5) (layer B.Cu) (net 2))
 (segment (start 130.7932 91.7296) (end 130.7932 94.4296) (width 0.5) (layer B.Cu) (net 2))
 (segment (start 130.7932 94.4296) (end 129.0932 96.1296) (width 0.5) (layer B.Cu) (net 2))
 (segment (start 129.0932 96.1296) (end 120.9932 96.1296) (width 0.5) (layer B.Cu) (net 2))
 (segment (start 119.1932 94.3296) (end 117.3932 94.3296) (width 0.5) (layer B.Cu) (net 2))
 (segment (start 120.9932 96.1296) (end 119.1932 94.3296) (width 0.5) (layer B.Cu) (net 2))
 (segment (start 133.8932 95.7296) (end 132.2932 95.7296) (width 0.5) (layer B.Cu) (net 2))
 (segment (start 130.9932 94.4296) (end 130.7932 94.4296) (width 0.5) (layer B.Cu) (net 2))
 (segment (start 132.2932 95.7296) (end 130.9932 94.4296) (width 0.5) (layer B.Cu) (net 2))
 (segment (start 116.26183 81.6296) (end 116.25583 81.6356) (width 0.5) (layer B.Cu) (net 1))
 (segment (start 117.3932 81.6296) (end 116.26183 81.6296) (width 0.5) (layer B.Cu) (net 1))
 (segment (start 116.25583 81.6356) (end 107.8484 81.6356) (width 0.5) (layer B.Cu) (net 1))
 (segment (start 107.8484 81.6356) (end 106.7308 82.7532) (width 0.5) (layer B.Cu) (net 1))
 (segment (start 106.7308 87.6972) (end 109.6932 90.6596) (width 0.5) (layer B.Cu) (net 1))
 (segment (start 106.7308 82.7532) (end 106.7308 87.6972) (width 0.5) (layer B.Cu) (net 1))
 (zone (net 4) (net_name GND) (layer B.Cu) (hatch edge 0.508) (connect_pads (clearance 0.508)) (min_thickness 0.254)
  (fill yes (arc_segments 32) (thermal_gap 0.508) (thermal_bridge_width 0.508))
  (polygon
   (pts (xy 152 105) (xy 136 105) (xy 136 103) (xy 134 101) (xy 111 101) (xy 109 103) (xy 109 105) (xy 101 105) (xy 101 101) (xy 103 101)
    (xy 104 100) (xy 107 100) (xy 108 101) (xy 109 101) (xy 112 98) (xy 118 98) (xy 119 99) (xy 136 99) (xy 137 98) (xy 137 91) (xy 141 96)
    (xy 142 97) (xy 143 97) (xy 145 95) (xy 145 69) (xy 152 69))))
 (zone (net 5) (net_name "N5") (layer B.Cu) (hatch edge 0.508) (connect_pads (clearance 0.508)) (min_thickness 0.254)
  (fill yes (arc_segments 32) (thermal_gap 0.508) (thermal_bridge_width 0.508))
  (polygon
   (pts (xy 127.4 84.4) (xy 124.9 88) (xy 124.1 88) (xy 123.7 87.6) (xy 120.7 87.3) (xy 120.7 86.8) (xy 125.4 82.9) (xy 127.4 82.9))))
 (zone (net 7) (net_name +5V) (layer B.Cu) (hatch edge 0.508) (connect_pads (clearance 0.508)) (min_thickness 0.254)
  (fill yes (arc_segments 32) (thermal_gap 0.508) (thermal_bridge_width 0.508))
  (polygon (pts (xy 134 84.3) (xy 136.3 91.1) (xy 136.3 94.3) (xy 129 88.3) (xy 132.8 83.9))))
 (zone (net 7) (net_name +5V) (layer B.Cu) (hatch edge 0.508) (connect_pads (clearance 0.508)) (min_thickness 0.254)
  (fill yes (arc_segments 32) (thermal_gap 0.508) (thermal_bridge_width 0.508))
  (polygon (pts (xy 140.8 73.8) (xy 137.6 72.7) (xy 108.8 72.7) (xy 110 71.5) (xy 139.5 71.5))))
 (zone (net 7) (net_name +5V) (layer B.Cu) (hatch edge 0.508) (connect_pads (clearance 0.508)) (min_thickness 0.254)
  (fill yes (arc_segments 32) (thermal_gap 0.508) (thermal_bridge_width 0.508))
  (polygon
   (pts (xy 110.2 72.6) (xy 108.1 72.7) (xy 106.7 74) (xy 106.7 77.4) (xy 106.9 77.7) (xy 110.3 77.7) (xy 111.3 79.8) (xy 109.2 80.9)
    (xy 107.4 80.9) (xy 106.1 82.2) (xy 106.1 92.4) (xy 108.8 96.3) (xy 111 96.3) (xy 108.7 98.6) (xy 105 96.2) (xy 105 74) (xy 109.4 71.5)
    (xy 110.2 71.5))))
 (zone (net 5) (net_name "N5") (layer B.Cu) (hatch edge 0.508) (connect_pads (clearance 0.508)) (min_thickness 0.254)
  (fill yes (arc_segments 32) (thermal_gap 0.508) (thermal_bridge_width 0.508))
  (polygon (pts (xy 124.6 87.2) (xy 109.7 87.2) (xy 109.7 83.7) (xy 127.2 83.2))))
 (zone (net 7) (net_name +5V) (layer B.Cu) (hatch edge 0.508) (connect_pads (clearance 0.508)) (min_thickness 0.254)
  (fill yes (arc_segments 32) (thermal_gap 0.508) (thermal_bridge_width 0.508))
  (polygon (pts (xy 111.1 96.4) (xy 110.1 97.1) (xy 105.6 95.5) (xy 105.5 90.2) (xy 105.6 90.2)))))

